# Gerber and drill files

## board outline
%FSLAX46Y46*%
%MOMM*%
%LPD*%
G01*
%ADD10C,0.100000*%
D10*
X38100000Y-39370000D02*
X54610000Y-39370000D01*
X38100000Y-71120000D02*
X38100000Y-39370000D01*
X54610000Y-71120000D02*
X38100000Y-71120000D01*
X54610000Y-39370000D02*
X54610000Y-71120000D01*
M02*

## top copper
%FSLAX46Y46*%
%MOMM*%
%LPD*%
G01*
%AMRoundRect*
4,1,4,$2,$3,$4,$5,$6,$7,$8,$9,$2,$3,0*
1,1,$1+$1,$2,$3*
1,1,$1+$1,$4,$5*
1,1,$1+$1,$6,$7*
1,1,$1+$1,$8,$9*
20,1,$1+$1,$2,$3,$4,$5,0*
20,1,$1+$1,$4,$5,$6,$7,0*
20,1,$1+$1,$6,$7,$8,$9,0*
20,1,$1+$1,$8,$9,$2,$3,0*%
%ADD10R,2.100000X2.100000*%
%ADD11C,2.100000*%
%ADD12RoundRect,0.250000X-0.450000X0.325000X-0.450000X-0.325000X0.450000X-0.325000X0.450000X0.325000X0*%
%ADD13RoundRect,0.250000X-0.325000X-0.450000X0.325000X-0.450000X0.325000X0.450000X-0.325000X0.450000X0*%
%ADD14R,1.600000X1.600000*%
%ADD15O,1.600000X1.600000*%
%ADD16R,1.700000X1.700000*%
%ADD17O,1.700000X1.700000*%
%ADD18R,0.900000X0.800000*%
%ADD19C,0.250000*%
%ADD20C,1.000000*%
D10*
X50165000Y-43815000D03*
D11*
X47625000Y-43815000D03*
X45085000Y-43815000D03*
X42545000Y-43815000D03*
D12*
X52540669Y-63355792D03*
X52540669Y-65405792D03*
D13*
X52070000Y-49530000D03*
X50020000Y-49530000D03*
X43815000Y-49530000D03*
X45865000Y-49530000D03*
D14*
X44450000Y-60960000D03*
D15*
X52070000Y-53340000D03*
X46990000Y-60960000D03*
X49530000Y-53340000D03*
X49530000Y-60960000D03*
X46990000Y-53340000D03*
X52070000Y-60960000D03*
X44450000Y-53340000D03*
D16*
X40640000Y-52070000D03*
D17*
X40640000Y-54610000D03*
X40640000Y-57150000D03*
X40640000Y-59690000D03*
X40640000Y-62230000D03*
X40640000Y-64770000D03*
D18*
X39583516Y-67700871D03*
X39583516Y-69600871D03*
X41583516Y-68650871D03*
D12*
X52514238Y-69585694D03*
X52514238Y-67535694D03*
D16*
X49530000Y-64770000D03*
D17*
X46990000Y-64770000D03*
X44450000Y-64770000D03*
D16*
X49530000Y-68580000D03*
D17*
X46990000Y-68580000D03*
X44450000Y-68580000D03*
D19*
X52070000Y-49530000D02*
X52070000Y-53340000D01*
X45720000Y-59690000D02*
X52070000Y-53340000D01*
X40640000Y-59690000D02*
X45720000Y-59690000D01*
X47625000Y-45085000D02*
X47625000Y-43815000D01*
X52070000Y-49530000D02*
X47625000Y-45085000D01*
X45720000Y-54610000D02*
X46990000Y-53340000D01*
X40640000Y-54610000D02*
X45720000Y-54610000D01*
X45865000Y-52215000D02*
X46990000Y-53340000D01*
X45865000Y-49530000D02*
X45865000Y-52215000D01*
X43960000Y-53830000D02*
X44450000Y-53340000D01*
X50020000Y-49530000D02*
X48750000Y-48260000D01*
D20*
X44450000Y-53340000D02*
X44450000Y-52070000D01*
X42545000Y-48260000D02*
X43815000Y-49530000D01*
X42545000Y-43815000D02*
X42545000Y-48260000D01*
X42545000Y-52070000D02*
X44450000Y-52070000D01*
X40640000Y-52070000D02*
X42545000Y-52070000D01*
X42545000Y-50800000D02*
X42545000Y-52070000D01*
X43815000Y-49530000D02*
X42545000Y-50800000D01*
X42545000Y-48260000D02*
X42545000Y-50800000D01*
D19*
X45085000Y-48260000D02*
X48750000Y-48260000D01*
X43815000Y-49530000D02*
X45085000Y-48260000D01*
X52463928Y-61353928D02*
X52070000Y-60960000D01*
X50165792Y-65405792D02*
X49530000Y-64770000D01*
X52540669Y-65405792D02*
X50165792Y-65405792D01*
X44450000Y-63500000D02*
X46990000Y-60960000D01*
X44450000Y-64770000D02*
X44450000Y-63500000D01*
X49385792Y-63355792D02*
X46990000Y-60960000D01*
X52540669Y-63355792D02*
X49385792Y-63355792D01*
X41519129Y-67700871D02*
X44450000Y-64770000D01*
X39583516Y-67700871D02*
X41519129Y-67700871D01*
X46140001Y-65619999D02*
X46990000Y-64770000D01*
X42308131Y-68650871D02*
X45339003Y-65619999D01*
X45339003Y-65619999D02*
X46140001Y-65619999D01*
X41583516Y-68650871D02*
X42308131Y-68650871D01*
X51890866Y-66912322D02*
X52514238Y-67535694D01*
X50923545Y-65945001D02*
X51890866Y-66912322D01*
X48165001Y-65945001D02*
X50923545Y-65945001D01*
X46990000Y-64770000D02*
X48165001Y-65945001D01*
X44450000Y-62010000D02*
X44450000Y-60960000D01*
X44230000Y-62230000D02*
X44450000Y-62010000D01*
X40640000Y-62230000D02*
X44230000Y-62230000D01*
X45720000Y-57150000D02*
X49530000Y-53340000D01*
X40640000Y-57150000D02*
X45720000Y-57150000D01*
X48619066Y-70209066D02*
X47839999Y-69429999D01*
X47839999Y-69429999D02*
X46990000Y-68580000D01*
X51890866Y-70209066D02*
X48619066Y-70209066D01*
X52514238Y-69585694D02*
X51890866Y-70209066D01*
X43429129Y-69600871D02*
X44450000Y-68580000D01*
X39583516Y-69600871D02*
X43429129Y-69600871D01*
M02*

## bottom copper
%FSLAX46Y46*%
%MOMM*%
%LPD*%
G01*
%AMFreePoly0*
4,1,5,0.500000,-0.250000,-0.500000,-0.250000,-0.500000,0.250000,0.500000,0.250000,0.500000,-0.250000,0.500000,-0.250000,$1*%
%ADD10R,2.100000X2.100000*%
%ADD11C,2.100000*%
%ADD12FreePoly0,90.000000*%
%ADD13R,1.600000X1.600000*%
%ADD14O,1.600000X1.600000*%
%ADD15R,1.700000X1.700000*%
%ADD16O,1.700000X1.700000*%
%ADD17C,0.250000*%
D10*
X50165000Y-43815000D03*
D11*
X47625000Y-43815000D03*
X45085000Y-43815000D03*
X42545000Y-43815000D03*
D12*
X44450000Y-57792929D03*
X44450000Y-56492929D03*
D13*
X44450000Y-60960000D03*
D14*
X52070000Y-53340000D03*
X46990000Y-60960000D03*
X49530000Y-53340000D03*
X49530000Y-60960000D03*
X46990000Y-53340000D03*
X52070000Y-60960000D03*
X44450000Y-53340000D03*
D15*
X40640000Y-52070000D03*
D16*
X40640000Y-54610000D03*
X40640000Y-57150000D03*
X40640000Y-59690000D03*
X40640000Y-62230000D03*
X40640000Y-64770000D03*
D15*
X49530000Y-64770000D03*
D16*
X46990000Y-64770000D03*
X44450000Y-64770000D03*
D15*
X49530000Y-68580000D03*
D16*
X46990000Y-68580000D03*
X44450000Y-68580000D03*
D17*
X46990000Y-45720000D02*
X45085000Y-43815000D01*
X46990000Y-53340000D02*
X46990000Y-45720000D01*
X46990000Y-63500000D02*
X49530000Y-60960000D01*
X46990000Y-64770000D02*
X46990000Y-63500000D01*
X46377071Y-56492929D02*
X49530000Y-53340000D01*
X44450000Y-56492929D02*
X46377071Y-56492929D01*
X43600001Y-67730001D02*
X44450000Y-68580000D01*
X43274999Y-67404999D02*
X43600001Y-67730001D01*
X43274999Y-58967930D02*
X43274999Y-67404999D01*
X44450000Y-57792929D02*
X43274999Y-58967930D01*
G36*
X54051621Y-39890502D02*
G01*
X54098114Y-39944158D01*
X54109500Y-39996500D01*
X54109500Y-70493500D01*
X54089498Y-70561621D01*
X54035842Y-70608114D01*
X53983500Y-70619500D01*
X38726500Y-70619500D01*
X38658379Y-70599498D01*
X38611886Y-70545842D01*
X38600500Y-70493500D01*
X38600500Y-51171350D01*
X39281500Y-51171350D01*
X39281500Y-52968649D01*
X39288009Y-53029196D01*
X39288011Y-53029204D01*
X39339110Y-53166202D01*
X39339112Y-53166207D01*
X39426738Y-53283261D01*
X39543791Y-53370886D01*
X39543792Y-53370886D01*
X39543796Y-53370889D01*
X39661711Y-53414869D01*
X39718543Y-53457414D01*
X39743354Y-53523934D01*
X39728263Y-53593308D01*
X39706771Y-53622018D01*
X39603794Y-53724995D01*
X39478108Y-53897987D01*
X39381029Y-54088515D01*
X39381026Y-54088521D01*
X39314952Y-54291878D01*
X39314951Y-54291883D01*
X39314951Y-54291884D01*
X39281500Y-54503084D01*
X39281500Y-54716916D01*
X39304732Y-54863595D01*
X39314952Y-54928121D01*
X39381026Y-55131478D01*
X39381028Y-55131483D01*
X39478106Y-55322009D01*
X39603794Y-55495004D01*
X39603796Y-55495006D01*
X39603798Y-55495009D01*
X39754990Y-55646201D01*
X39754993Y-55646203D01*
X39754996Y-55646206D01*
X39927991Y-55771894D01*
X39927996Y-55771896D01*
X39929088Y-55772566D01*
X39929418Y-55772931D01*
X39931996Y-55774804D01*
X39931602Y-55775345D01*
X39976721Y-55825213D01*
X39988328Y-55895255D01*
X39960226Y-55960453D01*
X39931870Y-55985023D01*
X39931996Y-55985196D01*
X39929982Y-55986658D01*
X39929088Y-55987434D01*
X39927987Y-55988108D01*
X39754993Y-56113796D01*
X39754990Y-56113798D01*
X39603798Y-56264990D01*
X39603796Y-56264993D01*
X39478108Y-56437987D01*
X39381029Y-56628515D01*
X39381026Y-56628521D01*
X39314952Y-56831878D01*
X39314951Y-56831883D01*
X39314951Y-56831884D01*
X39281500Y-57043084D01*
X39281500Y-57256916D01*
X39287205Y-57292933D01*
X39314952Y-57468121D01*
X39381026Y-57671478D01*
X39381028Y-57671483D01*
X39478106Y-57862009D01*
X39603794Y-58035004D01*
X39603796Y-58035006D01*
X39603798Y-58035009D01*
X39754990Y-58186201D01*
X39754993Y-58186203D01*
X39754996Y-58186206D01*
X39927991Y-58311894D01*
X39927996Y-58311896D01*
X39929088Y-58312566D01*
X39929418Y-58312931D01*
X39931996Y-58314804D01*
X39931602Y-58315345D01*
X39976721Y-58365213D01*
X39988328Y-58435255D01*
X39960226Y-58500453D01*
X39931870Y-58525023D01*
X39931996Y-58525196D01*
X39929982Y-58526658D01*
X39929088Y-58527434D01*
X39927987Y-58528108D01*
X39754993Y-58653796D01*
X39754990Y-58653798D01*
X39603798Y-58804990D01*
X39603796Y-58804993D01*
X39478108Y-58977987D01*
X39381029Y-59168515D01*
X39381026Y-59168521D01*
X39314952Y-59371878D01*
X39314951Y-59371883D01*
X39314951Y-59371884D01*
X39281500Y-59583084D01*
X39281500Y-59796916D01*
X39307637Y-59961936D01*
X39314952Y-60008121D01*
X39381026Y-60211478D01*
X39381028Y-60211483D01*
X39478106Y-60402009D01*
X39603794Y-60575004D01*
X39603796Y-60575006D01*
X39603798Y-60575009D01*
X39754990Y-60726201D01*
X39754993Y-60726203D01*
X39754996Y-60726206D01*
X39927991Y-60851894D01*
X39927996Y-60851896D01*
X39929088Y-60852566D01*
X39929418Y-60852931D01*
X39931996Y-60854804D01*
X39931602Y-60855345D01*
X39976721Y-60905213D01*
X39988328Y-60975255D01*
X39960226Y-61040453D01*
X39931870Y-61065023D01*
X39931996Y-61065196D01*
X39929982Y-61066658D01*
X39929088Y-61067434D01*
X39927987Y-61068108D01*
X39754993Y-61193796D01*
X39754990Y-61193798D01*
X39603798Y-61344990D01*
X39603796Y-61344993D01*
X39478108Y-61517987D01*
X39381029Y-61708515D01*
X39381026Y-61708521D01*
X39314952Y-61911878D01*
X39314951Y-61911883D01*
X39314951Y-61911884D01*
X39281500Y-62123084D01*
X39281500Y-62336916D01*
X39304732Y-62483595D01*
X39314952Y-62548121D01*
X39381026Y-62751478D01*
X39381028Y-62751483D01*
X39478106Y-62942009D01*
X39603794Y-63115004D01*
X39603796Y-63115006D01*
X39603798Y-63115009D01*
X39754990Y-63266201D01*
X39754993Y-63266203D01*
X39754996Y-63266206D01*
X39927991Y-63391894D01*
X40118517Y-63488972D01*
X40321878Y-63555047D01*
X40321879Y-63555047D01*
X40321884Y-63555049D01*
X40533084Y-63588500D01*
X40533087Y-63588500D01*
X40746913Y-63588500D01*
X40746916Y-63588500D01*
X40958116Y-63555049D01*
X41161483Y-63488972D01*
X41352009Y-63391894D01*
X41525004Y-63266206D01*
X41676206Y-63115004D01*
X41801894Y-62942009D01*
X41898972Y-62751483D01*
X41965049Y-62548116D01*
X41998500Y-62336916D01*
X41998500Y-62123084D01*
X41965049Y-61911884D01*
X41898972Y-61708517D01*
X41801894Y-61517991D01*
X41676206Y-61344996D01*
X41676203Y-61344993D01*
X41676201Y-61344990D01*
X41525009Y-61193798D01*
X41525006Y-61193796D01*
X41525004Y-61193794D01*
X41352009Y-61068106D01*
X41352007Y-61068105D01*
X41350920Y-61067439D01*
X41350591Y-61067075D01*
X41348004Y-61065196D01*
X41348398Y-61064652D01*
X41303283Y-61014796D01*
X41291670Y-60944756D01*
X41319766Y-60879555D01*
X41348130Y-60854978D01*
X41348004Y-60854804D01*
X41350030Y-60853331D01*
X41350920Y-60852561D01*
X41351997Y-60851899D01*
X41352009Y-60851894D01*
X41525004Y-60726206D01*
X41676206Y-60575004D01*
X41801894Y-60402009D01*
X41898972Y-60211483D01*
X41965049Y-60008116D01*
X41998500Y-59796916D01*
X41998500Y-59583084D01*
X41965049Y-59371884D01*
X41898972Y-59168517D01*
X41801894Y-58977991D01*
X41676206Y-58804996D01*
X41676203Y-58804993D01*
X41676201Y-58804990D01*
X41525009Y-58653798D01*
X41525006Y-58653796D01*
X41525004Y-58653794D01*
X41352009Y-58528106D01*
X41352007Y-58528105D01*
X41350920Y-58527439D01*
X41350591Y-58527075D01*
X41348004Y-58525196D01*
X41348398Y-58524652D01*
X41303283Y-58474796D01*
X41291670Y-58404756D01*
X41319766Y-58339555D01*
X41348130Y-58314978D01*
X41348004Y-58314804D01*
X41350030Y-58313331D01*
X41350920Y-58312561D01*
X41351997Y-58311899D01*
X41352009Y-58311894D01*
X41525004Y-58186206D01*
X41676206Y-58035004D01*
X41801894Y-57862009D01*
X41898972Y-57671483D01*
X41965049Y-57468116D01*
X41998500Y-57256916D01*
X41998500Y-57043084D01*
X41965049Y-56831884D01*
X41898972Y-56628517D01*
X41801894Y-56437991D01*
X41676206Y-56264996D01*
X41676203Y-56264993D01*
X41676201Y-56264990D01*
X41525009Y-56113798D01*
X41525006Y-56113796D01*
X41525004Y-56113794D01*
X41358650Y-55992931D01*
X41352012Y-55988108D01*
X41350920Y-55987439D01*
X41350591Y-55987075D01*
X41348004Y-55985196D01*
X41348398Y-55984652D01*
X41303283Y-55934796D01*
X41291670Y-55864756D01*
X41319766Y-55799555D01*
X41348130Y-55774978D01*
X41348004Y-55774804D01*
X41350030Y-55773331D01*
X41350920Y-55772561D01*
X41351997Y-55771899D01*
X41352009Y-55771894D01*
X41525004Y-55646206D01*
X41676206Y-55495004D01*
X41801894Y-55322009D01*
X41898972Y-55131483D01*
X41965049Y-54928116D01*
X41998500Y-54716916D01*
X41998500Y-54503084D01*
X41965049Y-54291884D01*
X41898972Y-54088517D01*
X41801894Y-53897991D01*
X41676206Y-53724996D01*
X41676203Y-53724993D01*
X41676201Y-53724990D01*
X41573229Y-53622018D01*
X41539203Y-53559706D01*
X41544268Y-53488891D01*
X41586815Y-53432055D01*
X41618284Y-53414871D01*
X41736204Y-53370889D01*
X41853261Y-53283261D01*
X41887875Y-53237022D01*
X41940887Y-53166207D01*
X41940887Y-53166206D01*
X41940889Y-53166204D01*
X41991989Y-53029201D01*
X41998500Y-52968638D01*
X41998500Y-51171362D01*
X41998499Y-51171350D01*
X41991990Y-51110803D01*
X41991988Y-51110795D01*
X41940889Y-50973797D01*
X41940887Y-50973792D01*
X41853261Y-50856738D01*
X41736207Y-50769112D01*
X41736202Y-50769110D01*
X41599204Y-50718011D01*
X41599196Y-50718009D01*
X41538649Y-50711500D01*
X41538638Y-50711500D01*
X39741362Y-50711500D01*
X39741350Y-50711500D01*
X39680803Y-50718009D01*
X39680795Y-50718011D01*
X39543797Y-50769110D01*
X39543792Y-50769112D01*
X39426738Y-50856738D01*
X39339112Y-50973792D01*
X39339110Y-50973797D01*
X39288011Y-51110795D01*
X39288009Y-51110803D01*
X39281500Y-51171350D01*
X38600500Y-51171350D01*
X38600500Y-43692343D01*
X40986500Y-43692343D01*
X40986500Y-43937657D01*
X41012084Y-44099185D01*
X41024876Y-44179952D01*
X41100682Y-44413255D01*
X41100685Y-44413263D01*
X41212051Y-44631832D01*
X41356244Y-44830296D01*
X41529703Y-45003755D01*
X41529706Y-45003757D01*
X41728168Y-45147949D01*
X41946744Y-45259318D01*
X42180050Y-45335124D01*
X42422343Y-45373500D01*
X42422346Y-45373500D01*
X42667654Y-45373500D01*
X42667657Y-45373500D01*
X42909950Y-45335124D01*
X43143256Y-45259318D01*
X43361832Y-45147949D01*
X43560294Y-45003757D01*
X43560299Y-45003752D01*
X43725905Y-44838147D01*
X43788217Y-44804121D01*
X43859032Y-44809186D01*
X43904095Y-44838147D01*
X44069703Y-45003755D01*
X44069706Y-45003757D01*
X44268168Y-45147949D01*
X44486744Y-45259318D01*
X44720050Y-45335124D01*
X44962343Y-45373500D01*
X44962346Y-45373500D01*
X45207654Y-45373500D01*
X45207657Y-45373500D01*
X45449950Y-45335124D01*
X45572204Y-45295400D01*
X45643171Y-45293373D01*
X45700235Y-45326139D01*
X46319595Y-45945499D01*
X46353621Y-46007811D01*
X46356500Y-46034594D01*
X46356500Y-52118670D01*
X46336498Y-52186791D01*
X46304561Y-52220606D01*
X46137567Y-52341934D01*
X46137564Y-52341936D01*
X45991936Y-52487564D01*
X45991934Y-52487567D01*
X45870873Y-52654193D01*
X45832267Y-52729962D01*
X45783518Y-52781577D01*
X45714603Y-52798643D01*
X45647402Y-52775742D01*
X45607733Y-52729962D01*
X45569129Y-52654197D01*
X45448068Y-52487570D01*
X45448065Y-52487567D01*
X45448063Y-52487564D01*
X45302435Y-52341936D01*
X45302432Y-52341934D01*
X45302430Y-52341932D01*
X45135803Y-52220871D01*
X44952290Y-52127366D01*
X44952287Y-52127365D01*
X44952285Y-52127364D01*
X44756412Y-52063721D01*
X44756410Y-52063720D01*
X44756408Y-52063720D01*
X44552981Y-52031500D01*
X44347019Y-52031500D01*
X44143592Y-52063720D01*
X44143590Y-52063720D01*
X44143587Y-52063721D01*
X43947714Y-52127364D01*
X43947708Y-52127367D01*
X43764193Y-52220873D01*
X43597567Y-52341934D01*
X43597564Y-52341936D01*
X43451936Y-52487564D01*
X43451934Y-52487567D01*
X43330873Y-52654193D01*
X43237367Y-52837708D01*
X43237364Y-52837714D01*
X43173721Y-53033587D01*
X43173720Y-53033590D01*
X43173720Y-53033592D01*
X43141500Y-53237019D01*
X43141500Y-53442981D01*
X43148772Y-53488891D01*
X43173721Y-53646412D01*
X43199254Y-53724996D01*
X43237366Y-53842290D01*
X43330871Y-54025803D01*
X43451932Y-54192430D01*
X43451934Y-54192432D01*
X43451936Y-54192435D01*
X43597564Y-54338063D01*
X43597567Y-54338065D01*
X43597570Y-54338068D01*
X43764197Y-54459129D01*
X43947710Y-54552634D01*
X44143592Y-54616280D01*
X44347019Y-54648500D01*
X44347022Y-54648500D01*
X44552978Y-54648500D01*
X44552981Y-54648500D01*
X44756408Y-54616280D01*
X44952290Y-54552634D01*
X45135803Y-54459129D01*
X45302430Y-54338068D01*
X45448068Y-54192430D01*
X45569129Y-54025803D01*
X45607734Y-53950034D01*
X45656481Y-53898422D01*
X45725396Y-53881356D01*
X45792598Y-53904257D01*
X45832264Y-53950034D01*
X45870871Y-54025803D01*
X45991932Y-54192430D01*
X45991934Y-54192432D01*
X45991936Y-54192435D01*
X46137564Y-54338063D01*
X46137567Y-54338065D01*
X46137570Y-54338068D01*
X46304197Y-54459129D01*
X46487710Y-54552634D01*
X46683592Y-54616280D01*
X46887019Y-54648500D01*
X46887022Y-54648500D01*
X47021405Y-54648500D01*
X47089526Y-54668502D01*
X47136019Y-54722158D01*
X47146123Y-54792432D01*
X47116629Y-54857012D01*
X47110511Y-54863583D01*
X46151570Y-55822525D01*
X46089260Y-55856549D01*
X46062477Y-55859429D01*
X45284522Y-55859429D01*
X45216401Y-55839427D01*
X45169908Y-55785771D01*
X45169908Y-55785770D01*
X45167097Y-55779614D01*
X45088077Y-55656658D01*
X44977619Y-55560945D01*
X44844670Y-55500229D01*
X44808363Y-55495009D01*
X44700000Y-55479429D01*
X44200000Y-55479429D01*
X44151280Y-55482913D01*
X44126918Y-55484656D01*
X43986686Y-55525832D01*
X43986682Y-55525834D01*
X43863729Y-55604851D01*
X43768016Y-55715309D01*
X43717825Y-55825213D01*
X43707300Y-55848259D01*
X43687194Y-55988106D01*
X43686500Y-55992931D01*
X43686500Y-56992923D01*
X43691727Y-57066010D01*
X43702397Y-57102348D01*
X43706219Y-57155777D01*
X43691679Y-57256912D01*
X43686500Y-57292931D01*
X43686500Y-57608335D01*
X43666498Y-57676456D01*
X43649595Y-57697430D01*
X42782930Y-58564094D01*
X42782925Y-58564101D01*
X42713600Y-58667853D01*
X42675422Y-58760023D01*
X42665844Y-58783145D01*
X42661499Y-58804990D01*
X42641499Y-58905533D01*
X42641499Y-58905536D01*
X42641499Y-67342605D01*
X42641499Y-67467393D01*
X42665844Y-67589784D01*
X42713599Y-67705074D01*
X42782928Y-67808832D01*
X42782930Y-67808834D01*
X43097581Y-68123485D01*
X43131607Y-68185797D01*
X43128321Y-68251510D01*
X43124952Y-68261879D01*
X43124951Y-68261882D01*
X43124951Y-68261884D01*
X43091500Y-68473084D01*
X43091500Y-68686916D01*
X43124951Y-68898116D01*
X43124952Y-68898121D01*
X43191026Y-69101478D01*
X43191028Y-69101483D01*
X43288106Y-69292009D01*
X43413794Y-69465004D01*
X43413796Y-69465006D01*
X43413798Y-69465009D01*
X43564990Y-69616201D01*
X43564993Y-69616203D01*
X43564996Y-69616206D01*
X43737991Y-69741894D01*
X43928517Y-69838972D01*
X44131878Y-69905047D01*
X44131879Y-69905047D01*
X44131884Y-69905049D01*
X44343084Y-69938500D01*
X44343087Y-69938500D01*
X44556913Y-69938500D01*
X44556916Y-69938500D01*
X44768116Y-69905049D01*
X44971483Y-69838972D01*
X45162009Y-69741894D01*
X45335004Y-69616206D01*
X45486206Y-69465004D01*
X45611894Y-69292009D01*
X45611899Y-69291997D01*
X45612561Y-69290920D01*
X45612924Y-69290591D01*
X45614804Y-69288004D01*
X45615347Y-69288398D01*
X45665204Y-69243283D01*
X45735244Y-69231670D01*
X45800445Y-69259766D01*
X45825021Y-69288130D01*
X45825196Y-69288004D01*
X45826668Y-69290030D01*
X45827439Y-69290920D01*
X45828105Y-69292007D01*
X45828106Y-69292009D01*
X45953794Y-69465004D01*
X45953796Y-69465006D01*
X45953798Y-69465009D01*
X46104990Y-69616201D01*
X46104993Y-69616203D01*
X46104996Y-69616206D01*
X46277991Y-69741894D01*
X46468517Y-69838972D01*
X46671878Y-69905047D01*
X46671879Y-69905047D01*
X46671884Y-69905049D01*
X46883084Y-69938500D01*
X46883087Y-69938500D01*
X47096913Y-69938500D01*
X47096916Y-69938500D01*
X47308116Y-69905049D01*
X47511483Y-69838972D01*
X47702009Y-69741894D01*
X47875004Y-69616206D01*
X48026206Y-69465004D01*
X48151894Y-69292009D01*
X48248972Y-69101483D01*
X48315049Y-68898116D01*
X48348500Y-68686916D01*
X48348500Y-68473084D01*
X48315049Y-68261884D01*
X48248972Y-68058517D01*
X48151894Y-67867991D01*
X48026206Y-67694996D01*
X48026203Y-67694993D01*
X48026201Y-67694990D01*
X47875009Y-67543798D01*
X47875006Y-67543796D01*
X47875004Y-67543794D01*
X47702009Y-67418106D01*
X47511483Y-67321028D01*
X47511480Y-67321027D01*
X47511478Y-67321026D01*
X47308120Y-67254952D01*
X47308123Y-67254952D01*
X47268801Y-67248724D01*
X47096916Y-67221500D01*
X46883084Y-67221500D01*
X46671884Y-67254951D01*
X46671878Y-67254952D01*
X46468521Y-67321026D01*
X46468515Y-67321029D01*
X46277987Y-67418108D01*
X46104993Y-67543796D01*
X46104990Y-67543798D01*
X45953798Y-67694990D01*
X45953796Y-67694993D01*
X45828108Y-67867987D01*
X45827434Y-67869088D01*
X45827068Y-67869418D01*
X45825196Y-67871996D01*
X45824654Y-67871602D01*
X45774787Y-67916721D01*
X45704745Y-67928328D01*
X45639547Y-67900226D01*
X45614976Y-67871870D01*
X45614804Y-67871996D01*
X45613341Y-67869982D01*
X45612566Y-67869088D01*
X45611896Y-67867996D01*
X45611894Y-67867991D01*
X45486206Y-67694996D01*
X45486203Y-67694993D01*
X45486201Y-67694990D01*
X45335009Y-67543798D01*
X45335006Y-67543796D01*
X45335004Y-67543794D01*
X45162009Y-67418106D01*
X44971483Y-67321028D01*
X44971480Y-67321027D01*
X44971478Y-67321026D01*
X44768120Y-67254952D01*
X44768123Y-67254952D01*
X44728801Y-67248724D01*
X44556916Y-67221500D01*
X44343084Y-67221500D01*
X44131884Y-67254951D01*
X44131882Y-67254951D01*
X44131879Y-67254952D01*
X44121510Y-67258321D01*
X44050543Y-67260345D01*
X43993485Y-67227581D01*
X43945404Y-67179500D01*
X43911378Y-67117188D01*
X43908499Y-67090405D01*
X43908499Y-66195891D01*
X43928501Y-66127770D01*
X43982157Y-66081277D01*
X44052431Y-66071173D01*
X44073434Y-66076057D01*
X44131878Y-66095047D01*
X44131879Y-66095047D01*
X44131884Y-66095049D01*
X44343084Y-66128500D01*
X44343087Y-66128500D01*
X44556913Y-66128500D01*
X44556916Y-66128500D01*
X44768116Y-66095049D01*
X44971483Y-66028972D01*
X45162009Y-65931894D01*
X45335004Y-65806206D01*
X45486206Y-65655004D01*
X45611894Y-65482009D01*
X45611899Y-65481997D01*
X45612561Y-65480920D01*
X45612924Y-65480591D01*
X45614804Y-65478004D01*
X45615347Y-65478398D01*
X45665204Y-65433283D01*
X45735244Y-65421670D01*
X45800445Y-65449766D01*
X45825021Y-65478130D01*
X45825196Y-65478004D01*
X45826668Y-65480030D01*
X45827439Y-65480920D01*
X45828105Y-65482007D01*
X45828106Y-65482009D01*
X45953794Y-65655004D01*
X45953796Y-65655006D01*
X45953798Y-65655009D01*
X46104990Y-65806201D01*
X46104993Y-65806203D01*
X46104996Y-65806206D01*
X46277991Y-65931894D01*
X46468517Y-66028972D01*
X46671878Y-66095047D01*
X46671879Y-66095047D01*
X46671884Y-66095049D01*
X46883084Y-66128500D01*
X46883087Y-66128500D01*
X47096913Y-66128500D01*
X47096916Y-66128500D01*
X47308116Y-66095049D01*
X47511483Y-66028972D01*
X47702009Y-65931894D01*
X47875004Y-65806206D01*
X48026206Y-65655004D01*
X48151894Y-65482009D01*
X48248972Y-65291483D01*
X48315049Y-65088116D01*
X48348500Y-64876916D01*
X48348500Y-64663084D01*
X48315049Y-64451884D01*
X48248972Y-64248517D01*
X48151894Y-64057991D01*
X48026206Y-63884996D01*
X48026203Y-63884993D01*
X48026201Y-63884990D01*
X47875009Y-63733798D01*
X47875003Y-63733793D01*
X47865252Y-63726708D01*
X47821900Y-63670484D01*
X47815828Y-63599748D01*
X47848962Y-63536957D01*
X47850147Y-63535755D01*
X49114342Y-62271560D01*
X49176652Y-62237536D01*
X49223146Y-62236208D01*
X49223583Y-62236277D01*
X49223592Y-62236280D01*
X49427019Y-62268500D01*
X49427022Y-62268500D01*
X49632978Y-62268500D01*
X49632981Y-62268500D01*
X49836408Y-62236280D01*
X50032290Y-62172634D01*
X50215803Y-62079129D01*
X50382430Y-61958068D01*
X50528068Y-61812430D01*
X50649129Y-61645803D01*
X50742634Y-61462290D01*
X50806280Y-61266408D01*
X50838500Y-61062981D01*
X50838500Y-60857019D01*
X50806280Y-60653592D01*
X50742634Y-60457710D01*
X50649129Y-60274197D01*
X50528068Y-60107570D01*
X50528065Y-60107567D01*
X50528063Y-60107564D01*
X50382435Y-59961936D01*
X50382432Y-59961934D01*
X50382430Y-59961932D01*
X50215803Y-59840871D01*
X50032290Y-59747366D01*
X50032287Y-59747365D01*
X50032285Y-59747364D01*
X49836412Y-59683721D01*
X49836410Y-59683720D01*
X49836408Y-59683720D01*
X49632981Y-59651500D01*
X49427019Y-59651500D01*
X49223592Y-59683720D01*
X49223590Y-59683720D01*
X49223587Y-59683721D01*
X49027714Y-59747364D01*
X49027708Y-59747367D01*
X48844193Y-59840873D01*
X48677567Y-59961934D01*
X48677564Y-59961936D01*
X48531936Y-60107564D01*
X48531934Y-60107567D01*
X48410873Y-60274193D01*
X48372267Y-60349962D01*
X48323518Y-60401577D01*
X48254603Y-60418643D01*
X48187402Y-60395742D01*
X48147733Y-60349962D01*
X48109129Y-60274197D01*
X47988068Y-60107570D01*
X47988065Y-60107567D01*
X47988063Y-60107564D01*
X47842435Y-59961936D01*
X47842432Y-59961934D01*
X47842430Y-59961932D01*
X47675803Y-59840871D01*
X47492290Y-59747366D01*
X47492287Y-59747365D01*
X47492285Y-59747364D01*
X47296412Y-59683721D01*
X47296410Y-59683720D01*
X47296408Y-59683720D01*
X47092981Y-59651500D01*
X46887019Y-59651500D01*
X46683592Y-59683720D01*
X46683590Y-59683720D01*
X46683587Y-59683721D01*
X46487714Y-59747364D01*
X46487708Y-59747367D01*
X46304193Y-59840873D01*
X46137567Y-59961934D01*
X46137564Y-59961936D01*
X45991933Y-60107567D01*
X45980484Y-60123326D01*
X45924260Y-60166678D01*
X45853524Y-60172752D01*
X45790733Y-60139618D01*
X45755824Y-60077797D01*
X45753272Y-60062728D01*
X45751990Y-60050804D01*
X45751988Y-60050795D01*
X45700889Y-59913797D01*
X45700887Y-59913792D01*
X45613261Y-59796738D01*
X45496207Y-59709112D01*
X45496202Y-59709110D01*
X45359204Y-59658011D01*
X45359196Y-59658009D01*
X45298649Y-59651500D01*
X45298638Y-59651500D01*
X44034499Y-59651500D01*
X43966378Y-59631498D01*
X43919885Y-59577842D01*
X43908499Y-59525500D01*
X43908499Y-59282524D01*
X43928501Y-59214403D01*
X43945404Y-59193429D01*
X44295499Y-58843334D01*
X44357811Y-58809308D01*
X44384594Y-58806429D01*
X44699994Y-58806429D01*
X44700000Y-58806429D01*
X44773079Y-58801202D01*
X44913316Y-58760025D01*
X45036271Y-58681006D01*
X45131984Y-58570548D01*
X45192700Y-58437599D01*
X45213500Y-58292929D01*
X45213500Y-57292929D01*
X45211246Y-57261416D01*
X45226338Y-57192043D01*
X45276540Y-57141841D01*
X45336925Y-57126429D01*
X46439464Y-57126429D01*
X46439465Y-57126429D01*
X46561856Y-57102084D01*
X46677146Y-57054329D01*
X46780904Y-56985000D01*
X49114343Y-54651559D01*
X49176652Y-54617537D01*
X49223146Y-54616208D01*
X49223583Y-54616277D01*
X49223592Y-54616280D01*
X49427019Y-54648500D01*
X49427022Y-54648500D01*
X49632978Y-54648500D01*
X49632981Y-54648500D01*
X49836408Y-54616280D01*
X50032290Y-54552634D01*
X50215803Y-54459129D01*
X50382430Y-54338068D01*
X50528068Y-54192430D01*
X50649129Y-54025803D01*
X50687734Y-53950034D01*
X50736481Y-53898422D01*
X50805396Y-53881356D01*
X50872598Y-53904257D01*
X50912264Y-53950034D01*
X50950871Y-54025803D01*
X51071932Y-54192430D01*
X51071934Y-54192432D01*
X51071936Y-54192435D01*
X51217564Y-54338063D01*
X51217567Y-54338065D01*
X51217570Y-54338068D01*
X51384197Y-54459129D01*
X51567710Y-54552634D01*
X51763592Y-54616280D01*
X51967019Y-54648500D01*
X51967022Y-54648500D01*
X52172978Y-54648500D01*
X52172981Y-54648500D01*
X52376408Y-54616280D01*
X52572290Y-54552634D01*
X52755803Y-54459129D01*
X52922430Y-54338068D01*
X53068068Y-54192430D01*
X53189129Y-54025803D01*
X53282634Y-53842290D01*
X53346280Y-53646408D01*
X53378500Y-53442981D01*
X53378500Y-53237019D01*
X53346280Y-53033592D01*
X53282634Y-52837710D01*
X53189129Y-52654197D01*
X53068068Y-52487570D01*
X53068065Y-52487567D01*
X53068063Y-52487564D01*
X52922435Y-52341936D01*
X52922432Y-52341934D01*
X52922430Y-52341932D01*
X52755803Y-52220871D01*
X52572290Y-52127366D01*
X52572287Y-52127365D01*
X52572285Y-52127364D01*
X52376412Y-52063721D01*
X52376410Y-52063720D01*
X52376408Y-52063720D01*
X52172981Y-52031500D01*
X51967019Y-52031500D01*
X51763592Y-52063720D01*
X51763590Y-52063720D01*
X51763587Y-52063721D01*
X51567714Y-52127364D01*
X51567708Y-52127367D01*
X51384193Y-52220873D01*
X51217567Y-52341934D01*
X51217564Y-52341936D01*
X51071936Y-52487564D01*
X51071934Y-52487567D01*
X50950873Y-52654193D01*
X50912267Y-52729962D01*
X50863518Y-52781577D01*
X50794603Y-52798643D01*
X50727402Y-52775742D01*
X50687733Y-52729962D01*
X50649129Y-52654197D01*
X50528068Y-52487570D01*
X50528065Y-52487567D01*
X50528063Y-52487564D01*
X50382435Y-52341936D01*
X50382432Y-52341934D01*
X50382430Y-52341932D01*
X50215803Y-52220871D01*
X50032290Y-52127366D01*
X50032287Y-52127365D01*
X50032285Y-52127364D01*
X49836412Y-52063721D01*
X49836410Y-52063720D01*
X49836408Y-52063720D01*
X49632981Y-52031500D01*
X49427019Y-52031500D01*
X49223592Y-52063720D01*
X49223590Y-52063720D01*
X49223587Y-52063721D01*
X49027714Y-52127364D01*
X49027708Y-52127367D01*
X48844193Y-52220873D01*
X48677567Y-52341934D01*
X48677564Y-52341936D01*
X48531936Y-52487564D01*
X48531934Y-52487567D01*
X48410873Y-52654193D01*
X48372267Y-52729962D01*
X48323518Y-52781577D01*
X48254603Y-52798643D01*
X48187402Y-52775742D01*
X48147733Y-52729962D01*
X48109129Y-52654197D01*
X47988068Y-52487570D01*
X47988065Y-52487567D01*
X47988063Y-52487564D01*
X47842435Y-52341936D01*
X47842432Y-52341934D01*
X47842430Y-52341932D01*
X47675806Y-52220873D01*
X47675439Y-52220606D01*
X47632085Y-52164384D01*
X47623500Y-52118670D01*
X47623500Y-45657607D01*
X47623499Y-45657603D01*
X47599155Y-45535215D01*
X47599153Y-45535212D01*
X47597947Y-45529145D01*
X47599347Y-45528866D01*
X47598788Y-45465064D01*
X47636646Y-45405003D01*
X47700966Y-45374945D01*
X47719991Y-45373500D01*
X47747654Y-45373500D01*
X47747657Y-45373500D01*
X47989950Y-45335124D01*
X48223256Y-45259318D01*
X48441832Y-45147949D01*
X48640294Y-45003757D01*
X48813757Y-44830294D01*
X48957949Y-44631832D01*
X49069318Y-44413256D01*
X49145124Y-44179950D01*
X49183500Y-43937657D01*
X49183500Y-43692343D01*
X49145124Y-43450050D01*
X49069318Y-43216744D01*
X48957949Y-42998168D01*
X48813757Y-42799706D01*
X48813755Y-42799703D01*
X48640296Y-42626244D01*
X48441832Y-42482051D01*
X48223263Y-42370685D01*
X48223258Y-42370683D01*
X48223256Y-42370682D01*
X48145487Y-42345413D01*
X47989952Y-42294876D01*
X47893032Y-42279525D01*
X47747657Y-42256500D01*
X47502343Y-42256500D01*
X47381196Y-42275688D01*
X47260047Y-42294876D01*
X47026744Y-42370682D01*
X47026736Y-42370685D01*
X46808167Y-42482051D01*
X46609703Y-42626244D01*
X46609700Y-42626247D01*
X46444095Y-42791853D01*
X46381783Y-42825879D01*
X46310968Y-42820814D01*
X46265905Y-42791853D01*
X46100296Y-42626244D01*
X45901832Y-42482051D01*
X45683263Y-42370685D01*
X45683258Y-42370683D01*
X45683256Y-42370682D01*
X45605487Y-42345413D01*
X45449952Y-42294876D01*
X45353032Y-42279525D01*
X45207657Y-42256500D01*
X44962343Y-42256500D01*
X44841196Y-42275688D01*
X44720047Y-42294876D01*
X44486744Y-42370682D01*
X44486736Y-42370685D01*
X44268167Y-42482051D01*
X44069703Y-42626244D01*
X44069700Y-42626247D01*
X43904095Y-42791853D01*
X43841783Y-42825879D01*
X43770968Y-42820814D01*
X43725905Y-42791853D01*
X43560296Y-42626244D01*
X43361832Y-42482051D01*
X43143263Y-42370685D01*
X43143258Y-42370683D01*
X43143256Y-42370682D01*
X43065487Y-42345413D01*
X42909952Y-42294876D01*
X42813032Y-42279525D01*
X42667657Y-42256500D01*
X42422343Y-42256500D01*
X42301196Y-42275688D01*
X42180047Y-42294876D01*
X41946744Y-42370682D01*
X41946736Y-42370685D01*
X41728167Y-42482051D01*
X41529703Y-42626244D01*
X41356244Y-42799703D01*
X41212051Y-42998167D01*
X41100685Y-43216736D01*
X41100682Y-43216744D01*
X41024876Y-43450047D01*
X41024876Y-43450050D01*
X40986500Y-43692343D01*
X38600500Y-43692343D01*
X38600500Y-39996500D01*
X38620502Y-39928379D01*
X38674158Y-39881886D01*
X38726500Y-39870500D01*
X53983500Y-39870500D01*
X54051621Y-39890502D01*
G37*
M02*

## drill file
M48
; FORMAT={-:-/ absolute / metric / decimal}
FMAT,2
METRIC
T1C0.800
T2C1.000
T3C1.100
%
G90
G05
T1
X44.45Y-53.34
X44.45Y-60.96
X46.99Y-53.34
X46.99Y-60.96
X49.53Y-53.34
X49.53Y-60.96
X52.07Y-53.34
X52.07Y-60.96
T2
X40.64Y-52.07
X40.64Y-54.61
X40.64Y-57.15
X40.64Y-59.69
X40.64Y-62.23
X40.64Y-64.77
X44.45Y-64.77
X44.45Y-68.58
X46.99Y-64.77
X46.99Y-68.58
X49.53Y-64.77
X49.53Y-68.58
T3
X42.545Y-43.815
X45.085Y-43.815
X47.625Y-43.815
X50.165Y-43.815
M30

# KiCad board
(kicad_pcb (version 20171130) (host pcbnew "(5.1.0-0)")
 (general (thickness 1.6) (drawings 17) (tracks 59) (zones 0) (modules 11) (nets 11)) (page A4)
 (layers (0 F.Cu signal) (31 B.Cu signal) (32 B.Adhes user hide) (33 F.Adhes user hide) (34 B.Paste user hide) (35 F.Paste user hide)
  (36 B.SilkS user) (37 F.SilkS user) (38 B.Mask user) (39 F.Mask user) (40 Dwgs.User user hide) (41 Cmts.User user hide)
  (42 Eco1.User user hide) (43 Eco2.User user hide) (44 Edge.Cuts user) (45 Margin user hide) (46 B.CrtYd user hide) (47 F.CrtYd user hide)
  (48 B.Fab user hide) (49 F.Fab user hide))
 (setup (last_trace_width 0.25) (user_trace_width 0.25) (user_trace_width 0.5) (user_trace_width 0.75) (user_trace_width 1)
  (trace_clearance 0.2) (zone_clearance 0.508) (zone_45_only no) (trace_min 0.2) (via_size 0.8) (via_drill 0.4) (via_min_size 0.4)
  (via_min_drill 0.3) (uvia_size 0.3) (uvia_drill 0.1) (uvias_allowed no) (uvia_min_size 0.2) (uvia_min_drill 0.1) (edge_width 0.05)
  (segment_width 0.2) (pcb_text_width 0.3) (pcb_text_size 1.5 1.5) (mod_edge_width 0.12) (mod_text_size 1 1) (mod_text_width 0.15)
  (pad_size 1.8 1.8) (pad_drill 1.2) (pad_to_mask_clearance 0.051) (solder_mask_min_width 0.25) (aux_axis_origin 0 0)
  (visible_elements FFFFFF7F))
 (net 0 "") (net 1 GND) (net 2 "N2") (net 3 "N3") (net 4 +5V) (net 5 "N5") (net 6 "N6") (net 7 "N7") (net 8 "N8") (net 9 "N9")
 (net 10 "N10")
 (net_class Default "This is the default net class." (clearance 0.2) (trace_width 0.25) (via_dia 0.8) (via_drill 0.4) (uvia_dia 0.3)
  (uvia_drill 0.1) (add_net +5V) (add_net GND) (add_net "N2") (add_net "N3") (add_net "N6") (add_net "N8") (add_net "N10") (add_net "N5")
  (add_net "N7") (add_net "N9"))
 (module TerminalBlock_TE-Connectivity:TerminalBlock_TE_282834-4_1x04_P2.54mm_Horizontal (layer F.Cu) (at 50.165 43.815 180)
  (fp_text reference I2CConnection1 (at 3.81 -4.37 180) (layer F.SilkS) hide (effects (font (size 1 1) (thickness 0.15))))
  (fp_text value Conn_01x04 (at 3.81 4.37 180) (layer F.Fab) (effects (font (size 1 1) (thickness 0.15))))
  (pad 1 thru_hole rect (at 0 0 180) (size 2.1 2.1) (drill 1.1) (layers *.Cu *.Mask) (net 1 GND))
  (pad 2 thru_hole circle (at 2.54 0 180) (size 2.1 2.1) (drill 1.1) (layers *.Cu *.Mask) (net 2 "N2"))
  (pad 3 thru_hole circle (at 5.08 0 180) (size 2.1 2.1) (drill 1.1) (layers *.Cu *.Mask) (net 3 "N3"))
  (pad 4 thru_hole circle (at 7.62 0 180) (size 2.1 2.1) (drill 1.1) (layers *.Cu *.Mask) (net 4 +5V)))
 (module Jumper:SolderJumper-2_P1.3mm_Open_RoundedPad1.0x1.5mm (layer B.Cu) (at 44.45 57.142929 90)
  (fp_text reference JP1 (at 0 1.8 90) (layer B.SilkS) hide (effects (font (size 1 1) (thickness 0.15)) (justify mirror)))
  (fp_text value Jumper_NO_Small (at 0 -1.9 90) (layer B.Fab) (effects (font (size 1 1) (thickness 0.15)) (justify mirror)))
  (pad 1 smd custom (at -0.65 0 90) (size 1 0.5) (layers B.Cu B.Mask) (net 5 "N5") (zone_connect 2)
   (options (clearance outline) (anchor rect)) (primitives))
  (pad 2 smd custom (at 0.65 0 90) (size 1 0.5) (layers B.Cu B.Mask) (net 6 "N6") (zone_connect 2)
   (options (clearance outline) (anchor rect)) (primitives)))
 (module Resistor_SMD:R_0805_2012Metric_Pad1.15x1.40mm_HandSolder (layer F.Cu) (at 52.540669 64.380792 270)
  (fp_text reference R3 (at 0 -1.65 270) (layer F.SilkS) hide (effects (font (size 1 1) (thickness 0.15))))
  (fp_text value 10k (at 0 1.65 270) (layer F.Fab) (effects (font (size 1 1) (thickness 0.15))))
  (pad 1 smd roundrect (at -1.025 0 270) (size 1.15 1.4) (layers F.Cu F.Paste F.Mask) (roundrect_rratio 0.217391) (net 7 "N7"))
  (pad 2 smd roundrect (at 1.025 0 270) (size 1.15 1.4) (layers F.Cu F.Paste F.Mask) (roundrect_rratio 0.217391) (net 1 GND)))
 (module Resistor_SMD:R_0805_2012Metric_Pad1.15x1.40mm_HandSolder (layer F.Cu) (at 51.045 49.53)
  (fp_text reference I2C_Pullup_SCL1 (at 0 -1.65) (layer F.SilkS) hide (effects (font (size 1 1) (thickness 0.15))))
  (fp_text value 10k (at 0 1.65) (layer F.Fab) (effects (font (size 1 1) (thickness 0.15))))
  (pad 2 smd roundrect (at 1.025 0) (size 1.15 1.4) (layers F.Cu F.Paste F.Mask) (roundrect_rratio 0.217391) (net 2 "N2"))
  (pad 1 smd roundrect (at -1.025 0) (size 1.15 1.4) (layers F.Cu F.Paste F.Mask) (roundrect_rratio 0.217391) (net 4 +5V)))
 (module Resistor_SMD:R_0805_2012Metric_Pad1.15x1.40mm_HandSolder (layer F.Cu) (at 44.84 49.53)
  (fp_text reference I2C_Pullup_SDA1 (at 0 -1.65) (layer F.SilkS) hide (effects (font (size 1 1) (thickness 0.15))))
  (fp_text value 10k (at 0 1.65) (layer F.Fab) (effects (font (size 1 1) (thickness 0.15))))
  (pad 1 smd roundrect (at -1.025 0) (size 1.15 1.4) (layers F.Cu F.Paste F.Mask) (roundrect_rratio 0.217391) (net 4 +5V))
  (pad 2 smd roundrect (at 1.025 0) (size 1.15 1.4) (layers F.Cu F.Paste F.Mask) (roundrect_rratio 0.217391) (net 3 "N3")))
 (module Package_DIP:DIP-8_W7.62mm (layer F.Cu) (at 44.45 60.96 90)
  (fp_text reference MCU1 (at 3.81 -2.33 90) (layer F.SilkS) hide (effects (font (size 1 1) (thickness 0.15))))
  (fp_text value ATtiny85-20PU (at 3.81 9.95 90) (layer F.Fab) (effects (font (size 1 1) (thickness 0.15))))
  (pad 1 thru_hole rect (at 0 0 90) (size 1.6 1.6) (drill 0.8) (layers *.Cu *.Mask) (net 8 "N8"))
  (pad 5 thru_hole oval (at 7.62 7.62 90) (size 1.6 1.6) (drill 0.8) (layers *.Cu *.Mask) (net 2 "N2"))
  (pad 2 thru_hole oval (at 0 2.54 90) (size 1.6 1.6) (drill 0.8) (layers *.Cu *.Mask) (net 7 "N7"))
  (pad 6 thru_hole oval (at 7.62 5.08 90) (size 1.6 1.6) (drill 0.8) (layers *.Cu *.Mask) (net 6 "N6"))
  (pad 3 thru_hole oval (at 0 5.08 90) (size 1.6 1.6) (drill 0.8) (layers *.Cu *.Mask) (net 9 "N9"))
  (pad 7 thru_hole oval (at 7.62 2.54 90) (size 1.6 1.6) (drill 0.8) (layers *.Cu *.Mask) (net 3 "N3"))
  (pad 4 thru_hole oval (at 0 7.62 90) (size 1.6 1.6) (drill 0.8) (layers *.Cu *.Mask) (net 1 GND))
  (pad 8 thru_hole oval (at 7.62 0 90) (size 1.6 1.6) (drill 0.8) (layers *.Cu *.Mask) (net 4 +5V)))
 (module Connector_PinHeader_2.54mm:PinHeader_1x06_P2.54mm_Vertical (layer F.Cu) (at 40.64 52.07)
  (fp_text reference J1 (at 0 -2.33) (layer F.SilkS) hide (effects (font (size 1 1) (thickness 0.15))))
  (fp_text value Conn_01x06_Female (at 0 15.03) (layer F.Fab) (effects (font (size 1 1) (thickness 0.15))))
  (pad 1 thru_hole rect (at 0 0) (size 1.7 1.7) (drill 1) (layers *.Cu *.Mask) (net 4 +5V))
  (pad 2 thru_hole oval (at 0 2.54) (size 1.7 1.7) (drill 1) (layers *.Cu *.Mask) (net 3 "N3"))
  (pad 3 thru_hole oval (at 0 5.08) (size 1.7 1.7) (drill 1) (layers *.Cu *.Mask) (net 6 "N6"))
  (pad 4 thru_hole oval (at 0 7.62) (size 1.7 1.7) (drill 1) (layers *.Cu *.Mask) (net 2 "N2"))
  (pad 5 thru_hole oval (at 0 10.16) (size 1.7 1.7) (drill 1) (layers *.Cu *.Mask) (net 8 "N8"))
  (pad 6 thru_hole oval (at 0 12.7) (size 1.7 1.7) (drill 1) (layers *.Cu *.Mask) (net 1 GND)))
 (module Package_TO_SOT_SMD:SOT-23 (layer F.Cu) (at 40.583516 68.650871)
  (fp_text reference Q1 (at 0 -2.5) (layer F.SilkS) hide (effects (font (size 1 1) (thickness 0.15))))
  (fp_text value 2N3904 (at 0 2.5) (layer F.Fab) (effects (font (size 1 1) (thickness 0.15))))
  (pad 1 smd rect (at -1 -0.95) (size 0.9 0.8) (layers F.Cu F.Paste F.Mask) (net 7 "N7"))
  (pad 2 smd rect (at -1 0.95) (size 0.9 0.8) (layers F.Cu F.Paste F.Mask) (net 5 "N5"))
  (pad 3 smd rect (at 1 0) (size 0.9 0.8) (layers F.Cu F.Paste F.Mask) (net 9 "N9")))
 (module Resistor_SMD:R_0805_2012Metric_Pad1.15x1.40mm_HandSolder (layer F.Cu) (at 52.514238 68.560694 270)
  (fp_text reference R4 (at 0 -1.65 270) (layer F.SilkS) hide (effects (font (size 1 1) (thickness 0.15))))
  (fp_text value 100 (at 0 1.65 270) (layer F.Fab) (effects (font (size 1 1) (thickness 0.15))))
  (pad 2 smd roundrect (at 1.025 0 270) (size 1.15 1.4) (layers F.Cu F.Paste F.Mask) (roundrect_rratio 0.217391) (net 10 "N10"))
  (pad 1 smd roundrect (at -1.025 0 270) (size 1.15 1.4) (layers F.Cu F.Paste F.Mask) (roundrect_rratio 0.217391) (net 9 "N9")))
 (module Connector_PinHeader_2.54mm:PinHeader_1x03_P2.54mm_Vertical (layer F.Cu) (at 49.53 64.77 270)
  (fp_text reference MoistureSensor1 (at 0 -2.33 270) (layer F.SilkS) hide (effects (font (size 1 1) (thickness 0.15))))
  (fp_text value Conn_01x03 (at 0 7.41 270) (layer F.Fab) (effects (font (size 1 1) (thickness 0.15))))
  (pad 1 thru_hole rect (at 0 0 270) (size 1.7 1.7) (drill 1) (layers *.Cu *.Mask) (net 1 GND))
  (pad 2 thru_hole oval (at 0 2.54 270) (size 1.7 1.7) (drill 1) (layers *.Cu *.Mask) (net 9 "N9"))
  (pad 3 thru_hole oval (at 0 5.08 270) (size 1.7 1.7) (drill 1) (layers *.Cu *.Mask) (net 7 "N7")))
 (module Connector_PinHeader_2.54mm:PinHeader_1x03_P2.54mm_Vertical (layer F.Cu) (at 49.53 68.58 270)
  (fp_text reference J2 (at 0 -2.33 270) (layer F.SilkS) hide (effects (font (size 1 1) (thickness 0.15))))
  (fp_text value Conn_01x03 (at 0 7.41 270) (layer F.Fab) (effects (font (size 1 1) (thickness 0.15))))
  (pad 1 thru_hole rect (at 0 0 270) (size 1.7 1.7) (drill 1) (layers *.Cu *.Mask) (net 1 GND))
  (pad 2 thru_hole oval (at 0 2.54 270) (size 1.7 1.7) (drill 1) (layers *.Cu *.Mask) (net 10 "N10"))
  (pad 3 thru_hole oval (at 0 5.08 270) (size 1.7 1.7) (drill 1) (layers *.Cu *.Mask) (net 5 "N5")))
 (gr_line (start 38.1 39.37) (end 54.61 39.37) (layer Edge.Cuts) (width 0.1))
 (gr_line (start 38.1 71.12) (end 38.1 39.37) (layer Edge.Cuts) (width 0.1))
 (gr_line (start 54.61 71.12) (end 38.1 71.12) (layer Edge.Cuts) (width 0.1))
 (gr_line (start 54.61 39.37) (end 54.61 71.12) (layer Edge.Cuts) (width 0.1))
 (segment (start 52.07 49.53) (end 52.07 53.34) (width 0.25) (layer F.Cu) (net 2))
 (segment (start 45.72 59.69) (end 52.07 53.34) (width 0.25) (layer F.Cu) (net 2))
 (segment (start 40.64 59.69) (end 45.72 59.69) (width 0.25) (layer F.Cu) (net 2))
 (segment (start 47.625 45.085) (end 47.625 43.815) (width 0.25) (layer F.Cu) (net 2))
 (segment (start 52.07 49.53) (end 47.625 45.085) (width 0.25) (layer F.Cu) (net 2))
 (segment (start 45.72 54.61) (end 46.99 53.34) (width 0.25) (layer F.Cu) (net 3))
 (segment (start 40.64 54.61) (end 45.72 54.61) (width 0.25) (layer F.Cu) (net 3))
 (segment (start 46.99 45.72) (end 45.085 43.815) (width 0.25) (layer B.Cu) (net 3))
 (segment (start 46.99 53.34) (end 46.99 45.72) (width 0.25) (layer B.Cu) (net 3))
 (segment (start 45.865 52.215) (end 46.99 53.34) (width 0.25) (layer F.Cu) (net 3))
 (segment (start 45.865 49.53) (end 45.865 52.215) (width 0.25) (layer F.Cu) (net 3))
 (segment (start 43.96 53.83) (end 44.45 53.34) (width 0.25) (layer F.Cu) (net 4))
 (segment (start 50.02 49.53) (end 48.75 48.26) (width 0.25) (layer F.Cu) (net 4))
 (segment (start 44.45 53.34) (end 44.45 52.07) (width 1) (layer F.Cu) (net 4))
 (segment (start 42.545 48.26) (end 43.815 49.53) (width 1) (layer F.Cu) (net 4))
 (segment (start 42.545 43.815) (end 42.545 48.26) (width 1) (layer F.Cu) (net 4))
 (segment (start 42.545 52.07) (end 44.45 52.07) (width 1) (layer F.Cu) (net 4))
 (segment (start 40.64 52.07) (end 42.545 52.07) (width 1) (layer F.Cu) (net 4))
 (segment (start 42.545 50.8) (end 42.545 52.07) (width 1) (layer F.Cu) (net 4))
 (segment (start 43.815 49.53) (end 42.545 50.8) (width 1) (layer F.Cu) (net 4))
 (segment (start 42.545 48.26) (end 42.545 50.8) (width 1) (layer F.Cu) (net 4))
 (segment (start 45.085 48.26) (end 48.75 48.26) (width 0.25) (layer F.Cu) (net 4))
 (segment (start 43.815 49.53) (end 45.085 48.26) (width 0.25) (layer F.Cu) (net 4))
 (segment (start 52.463928 61.353928) (end 52.07 60.96) (width 0.25) (layer F.Cu) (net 1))
 (segment (start 50.165792 65.405792) (end 49.53 64.77) (width 0.25) (layer F.Cu) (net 1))
 (segment (start 52.540669 65.405792) (end 50.165792 65.405792) (width 0.25) (layer F.Cu) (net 1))
 (segment (start 44.45 63.5) (end 46.99 60.96) (width 0.25) (layer F.Cu) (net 7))
 (segment (start 44.45 64.77) (end 44.45 63.5) (width 0.25) (layer F.Cu) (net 7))
 (segment (start 49.385792 63.355792) (end 46.99 60.96) (width 0.25) (layer F.Cu) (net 7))
 (segment (start 52.540669 63.355792) (end 49.385792 63.355792) (width 0.25) (layer F.Cu) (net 7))
 (segment (start 41.519129 67.700871) (end 44.45 64.77) (width 0.25) (layer F.Cu) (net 7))
 (segment (start 39.583516 67.700871) (end 41.519129 67.700871) (width 0.25) (layer F.Cu) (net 7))
 (segment (start 46.99 63.5) (end 49.53 60.96) (width 0.25) (layer B.Cu) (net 9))
 (segment (start 46.99 64.77) (end 46.99 63.5) (width 0.25) (layer B.Cu) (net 9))
 (segment (start 46.140001 65.619999) (end 46.99 64.77) (width 0.25) (layer F.Cu) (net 9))
 (segment (start 42.308131 68.650871) (end 45.339003 65.619999) (width 0.25) (layer F.Cu) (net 9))
 (segment (start 45.339003 65.619999) (end 46.140001 65.619999) (width 0.25) (layer F.Cu) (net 9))
 (segment (start 41.583516 68.650871) (end 42.308131 68.650871) (width 0.25) (layer F.Cu) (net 9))
 (segment (start 51.890866 66.912322) (end 52.514238 67.535694) (width 0.25) (layer F.Cu) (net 9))
 (segment (start 50.923545 65.945001) (end 51.890866 66.912322) (width 0.25) (layer F.Cu) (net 9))
 (segment (start 48.165001 65.945001) (end 50.923545 65.945001) (width 0.25) (layer F.Cu) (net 9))
 (segment (start 46.99 64.77) (end 48.165001 65.945001) (width 0.25) (layer F.Cu) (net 9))
 (segment (start 44.45 62.01) (end 44.45 60.96) (width 0.25) (layer F.Cu) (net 8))
 (segment (start 44.23 62.23) (end 44.45 62.01) (width 0.25) (layer F.Cu) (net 8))
 (segment (start 40.64 62.23) (end 44.23 62.23) (width 0.25) (layer F.Cu) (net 8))
 (segment (start 45.72 57.15) (end 49.53 53.34) (width 0.25) (layer F.Cu) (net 6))
 (segment (start 40.64 57.15) (end 45.72 57.15) (width 0.25) (layer F.Cu) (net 6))
 (segment (start 46.377071 56.492929) (end 49.53 53.34) (width 0.25) (layer B.Cu) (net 6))
 (segment (start 44.45 56.492929) (end 46.377071 56.492929) (width 0.25) (layer B.Cu) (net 6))
 (segment (start 48.619066 70.209066) (end 47.839999 69.429999) (width 0.25) (layer F.Cu) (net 10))
 (segment (start 47.839999 69.429999) (end 46.99 68.58) (width 0.25) (layer F.Cu) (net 10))
 (segment (start 51.890866 70.209066) (end 48.619066 70.209066) (width 0.25) (layer F.Cu) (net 10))
 (segment (start 52.514238 69.585694) (end 51.890866 70.209066) (width 0.25) (layer F.Cu) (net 10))
 (segment (start 43.600001 67.730001) (end 44.45 68.58) (width 0.25) (layer B.Cu) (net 5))
 (segment (start 43.274999 67.404999) (end 43.600001 67.730001) (width 0.25) (layer B.Cu) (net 5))
 (segment (start 43.274999 58.96793) (end 43.274999 67.404999) (width 0.25) (layer B.Cu) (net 5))
 (segment (start 44.45 57.792929) (end 43.274999 58.96793) (width 0.25) (layer B.Cu) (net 5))
 (segment (start 43.429129 69.600871) (end 44.45 68.58) (width 0.25) (layer F.Cu) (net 5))
 (segment (start 39.583516 69.600871) (end 43.429129 69.600871) (width 0.25) (layer F.Cu) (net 5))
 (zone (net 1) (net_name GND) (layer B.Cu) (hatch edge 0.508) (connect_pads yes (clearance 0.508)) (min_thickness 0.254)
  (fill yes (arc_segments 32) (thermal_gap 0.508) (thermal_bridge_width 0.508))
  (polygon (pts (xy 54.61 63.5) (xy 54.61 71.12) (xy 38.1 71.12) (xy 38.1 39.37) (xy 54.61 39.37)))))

